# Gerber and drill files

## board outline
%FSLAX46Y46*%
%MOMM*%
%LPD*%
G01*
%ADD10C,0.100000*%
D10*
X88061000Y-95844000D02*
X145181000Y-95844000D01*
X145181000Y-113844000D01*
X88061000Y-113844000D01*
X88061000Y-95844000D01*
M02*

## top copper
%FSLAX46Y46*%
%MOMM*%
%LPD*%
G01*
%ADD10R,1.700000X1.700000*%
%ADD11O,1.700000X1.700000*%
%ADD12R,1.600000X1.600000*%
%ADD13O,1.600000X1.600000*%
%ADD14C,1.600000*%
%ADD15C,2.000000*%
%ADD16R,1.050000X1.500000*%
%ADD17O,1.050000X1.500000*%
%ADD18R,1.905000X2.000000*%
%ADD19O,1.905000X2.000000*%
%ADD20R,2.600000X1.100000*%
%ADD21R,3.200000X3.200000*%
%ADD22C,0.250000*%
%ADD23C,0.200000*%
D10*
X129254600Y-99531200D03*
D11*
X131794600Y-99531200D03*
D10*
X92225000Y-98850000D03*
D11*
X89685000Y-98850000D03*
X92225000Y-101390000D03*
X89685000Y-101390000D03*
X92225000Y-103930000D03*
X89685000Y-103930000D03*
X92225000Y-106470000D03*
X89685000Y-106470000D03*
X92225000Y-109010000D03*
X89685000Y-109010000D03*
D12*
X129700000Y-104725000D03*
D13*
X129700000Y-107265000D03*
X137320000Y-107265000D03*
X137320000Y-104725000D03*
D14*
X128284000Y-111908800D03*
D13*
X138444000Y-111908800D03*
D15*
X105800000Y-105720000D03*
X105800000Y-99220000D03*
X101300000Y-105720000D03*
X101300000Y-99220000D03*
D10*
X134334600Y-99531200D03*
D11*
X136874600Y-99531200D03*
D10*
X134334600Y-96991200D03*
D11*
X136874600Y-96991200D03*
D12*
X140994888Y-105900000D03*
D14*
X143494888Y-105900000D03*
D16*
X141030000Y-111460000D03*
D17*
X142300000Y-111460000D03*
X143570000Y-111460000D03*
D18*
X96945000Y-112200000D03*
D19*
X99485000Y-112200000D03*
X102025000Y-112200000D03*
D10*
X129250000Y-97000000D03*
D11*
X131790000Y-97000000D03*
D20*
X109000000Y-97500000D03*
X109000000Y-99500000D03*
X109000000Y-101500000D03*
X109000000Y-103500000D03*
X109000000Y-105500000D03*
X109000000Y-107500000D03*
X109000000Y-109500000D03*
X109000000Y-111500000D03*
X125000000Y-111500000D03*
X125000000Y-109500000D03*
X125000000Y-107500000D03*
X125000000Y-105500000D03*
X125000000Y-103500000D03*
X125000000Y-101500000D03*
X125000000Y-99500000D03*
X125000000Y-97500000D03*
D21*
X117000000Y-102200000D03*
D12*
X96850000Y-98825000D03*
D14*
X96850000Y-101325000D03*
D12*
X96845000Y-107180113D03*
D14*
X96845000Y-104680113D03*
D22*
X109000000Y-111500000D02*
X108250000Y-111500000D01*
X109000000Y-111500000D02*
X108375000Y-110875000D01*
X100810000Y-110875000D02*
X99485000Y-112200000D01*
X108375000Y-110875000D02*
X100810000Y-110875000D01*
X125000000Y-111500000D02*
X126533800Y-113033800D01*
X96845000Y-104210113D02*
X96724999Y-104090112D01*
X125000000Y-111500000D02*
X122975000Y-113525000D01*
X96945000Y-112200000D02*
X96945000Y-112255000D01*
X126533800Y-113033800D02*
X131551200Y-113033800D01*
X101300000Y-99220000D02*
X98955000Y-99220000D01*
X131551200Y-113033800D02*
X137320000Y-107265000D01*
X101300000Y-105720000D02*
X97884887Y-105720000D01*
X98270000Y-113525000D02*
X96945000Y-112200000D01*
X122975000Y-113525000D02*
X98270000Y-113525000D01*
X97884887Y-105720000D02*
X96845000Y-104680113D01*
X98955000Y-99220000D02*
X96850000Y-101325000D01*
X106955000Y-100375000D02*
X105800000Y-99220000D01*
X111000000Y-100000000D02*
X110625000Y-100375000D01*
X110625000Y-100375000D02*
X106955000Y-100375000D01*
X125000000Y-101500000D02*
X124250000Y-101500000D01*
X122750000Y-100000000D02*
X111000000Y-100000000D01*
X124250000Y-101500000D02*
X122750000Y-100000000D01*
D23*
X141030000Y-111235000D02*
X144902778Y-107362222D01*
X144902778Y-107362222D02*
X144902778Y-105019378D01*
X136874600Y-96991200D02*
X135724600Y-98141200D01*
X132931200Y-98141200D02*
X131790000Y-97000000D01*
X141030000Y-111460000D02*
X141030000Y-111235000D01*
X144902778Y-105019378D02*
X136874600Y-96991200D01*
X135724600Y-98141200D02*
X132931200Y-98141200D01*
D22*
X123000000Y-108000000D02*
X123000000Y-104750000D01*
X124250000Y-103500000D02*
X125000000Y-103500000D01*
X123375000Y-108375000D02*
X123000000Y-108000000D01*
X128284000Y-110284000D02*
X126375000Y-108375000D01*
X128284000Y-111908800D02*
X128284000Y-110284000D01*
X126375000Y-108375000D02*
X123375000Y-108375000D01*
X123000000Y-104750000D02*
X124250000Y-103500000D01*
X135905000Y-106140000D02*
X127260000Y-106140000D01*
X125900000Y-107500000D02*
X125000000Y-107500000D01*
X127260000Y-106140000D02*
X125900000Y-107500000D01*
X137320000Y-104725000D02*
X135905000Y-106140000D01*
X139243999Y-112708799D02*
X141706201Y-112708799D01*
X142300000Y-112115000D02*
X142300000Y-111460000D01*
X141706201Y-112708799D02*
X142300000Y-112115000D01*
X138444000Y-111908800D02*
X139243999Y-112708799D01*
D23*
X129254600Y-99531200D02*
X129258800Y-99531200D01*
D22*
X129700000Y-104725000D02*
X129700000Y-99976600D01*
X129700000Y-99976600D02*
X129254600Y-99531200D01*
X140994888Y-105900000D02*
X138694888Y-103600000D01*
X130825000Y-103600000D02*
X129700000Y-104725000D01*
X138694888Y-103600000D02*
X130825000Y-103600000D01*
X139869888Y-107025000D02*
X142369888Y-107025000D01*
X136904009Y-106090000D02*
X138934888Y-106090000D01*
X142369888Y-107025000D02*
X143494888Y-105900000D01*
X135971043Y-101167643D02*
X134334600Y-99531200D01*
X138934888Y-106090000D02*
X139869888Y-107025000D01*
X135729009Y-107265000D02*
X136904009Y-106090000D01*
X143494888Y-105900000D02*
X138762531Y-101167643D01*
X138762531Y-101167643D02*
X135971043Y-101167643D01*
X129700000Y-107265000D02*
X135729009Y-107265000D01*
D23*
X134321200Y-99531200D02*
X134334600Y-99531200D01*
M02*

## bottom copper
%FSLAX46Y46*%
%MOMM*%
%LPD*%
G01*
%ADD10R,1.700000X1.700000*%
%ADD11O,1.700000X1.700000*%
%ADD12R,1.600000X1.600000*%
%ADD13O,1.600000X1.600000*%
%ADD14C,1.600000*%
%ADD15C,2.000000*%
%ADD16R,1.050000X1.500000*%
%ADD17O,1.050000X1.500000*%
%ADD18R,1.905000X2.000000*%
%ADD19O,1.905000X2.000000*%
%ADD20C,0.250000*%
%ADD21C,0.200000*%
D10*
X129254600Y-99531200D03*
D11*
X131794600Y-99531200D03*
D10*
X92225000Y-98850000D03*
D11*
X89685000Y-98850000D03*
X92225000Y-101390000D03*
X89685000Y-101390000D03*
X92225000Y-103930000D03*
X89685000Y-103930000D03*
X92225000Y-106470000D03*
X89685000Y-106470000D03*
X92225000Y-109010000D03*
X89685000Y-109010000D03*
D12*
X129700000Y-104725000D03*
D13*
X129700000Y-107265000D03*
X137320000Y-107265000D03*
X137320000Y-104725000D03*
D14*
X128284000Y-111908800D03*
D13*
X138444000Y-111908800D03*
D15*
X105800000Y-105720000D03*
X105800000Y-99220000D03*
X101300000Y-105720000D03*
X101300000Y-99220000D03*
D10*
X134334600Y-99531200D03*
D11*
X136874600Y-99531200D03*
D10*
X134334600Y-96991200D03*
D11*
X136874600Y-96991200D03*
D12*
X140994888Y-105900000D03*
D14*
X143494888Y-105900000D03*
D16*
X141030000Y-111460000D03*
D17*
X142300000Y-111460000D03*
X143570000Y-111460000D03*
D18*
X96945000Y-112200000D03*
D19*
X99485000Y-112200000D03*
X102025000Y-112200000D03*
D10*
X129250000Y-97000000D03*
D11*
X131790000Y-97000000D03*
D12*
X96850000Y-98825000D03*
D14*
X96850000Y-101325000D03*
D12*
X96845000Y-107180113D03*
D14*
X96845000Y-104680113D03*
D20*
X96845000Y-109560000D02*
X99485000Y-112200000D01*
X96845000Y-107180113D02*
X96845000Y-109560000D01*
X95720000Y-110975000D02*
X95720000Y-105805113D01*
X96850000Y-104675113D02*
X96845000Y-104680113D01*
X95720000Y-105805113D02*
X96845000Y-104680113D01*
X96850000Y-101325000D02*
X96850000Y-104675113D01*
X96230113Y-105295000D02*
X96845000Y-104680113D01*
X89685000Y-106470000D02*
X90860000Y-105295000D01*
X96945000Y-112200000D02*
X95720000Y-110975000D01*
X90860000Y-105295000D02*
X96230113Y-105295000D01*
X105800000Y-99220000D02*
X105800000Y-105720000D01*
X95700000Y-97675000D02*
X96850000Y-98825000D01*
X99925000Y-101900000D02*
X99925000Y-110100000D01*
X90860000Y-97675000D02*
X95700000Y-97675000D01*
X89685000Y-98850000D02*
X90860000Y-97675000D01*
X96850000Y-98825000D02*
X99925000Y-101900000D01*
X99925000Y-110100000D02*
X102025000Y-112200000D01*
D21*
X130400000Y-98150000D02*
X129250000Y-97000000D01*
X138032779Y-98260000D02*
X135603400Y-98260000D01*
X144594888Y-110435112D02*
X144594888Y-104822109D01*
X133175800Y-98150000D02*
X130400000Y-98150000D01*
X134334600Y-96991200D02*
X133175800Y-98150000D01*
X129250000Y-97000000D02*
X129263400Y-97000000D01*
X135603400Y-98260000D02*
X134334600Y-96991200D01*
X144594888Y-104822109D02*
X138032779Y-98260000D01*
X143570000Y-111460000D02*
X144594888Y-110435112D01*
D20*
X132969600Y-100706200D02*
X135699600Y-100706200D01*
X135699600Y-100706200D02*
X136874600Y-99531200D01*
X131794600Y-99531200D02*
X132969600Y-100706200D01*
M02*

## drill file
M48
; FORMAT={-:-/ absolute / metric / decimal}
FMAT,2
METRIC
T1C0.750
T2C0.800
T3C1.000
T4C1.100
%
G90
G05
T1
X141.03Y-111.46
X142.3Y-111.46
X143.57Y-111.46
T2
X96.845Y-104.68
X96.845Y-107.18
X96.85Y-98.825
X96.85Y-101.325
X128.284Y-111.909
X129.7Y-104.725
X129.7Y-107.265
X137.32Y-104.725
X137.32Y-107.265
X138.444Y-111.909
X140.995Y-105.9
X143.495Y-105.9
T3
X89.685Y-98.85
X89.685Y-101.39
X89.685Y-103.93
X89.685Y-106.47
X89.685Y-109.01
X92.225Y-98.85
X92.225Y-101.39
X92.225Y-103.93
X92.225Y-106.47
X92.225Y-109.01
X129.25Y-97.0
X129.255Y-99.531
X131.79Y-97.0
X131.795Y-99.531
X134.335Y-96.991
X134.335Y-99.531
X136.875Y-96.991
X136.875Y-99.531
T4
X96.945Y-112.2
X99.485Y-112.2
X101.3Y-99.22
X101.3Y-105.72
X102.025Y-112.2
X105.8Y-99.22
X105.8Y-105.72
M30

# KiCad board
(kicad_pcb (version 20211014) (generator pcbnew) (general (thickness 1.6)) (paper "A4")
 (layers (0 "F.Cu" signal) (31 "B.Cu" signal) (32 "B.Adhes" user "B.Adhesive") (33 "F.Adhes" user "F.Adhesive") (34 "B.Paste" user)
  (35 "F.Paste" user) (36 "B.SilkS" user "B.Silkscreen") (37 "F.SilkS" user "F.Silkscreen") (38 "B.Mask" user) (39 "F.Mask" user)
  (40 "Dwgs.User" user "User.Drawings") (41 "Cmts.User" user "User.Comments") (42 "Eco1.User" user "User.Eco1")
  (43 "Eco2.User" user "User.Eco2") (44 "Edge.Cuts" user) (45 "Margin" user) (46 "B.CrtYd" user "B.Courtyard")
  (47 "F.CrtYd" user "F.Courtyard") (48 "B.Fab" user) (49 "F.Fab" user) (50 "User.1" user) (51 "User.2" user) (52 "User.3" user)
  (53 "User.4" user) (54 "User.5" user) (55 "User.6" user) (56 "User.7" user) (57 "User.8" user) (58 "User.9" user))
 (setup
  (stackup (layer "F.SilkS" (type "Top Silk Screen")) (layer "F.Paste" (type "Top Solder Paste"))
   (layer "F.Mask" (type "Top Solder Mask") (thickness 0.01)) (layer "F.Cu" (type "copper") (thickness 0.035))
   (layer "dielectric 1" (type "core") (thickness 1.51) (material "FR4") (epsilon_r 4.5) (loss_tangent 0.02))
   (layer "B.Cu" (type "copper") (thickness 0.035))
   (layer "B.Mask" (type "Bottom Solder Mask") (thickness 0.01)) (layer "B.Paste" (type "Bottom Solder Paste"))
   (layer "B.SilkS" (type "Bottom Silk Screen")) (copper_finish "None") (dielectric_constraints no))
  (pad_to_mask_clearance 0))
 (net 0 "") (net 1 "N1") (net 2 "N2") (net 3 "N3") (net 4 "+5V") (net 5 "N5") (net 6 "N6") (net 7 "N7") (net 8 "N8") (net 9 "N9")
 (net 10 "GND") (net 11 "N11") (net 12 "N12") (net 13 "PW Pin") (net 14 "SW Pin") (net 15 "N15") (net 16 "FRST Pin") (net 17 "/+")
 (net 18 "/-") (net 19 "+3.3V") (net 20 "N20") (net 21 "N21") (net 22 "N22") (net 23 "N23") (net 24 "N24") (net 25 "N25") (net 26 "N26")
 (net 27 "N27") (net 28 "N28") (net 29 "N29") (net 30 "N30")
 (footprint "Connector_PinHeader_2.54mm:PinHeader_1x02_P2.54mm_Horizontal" (layer "F.Cu") (at 129.2546 99.5312 90)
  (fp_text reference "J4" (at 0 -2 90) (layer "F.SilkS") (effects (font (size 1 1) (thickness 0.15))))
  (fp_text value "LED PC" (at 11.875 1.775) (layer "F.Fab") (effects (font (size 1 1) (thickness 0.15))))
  (pad "1" thru_hole rect (at 0 0 90) (size 1.7 1.7) (drill 1) (layers *.Cu *.Mask) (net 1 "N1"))
  (pad "2" thru_hole oval (at 0 2.54 90) (size 1.7 1.7) (drill 1) (layers *.Cu *.Mask) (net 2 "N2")))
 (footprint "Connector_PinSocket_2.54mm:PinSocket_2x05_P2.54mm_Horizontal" (layer "F.Cu") (at 92.225 98.85)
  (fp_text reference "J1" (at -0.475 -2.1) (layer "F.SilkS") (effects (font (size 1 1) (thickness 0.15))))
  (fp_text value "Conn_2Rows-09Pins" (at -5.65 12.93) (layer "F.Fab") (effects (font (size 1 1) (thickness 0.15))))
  (pad "1" thru_hole rect (at 0 0) (size 1.7 1.7) (drill 1) (layers *.Cu *.Mask) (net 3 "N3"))
  (pad "2" thru_hole oval (at -2.54 0) (size 1.7 1.7) (drill 1) (layers *.Cu *.Mask) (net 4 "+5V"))
  (pad "3" thru_hole oval (at 0 2.54) (size 1.7 1.7) (drill 1) (layers *.Cu *.Mask) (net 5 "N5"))
  (pad "4" thru_hole oval (at -2.54 2.54) (size 1.7 1.7) (drill 1) (layers *.Cu *.Mask) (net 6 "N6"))
  (pad "5" thru_hole oval (at 0 5.08) (size 1.7 1.7) (drill 1) (layers *.Cu *.Mask) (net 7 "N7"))
  (pad "6" thru_hole oval (at -2.54 5.08) (size 1.7 1.7) (drill 1) (layers *.Cu *.Mask) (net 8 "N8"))
  (pad "7" thru_hole oval (at 0 7.62) (size 1.7 1.7) (drill 1) (layers *.Cu *.Mask) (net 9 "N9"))
  (pad "8" thru_hole oval (at -2.54 7.62) (size 1.7 1.7) (drill 1) (layers *.Cu *.Mask) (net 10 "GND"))
  (pad "9" thru_hole oval (at 0 10.16) (size 1.7 1.7) (drill 1) (layers *.Cu *.Mask) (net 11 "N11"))
  (pad "10" thru_hole oval (at -2.54 10.16) (size 1.7 1.7) (drill 1) (layers *.Cu *.Mask)))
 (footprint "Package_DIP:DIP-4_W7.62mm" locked (layer "F.Cu") (at 129.7 104.725)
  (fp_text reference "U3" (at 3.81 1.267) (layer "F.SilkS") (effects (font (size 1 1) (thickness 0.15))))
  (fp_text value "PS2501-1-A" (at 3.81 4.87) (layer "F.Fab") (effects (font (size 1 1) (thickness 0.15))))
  (pad "1" thru_hole rect locked (at 0 0) (size 1.6 1.6) (drill 0.8) (layers *.Cu *.Mask) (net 1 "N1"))
  (pad "2" thru_hole oval locked (at 0 2.54) (size 1.6 1.6) (drill 0.8) (layers *.Cu *.Mask) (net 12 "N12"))
  (pad "3" thru_hole oval locked (at 7.62 2.54) (size 1.6 1.6) (drill 0.8) (layers *.Cu *.Mask) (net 10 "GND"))
  (pad "4" thru_hole oval locked (at 7.62 0) (size 1.6 1.6) (drill 0.8) (layers *.Cu *.Mask) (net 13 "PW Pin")))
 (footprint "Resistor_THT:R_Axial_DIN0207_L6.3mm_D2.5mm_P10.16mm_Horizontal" (layer "F.Cu") (at 128.284 111.9088)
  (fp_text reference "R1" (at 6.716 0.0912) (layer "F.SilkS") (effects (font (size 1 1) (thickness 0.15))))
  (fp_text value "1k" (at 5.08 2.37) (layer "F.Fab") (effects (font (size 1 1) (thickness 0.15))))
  (pad "1" thru_hole circle (at 0 0) (size 1.6 1.6) (drill 0.8) (layers *.Cu *.Mask) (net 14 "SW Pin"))
  (pad "2" thru_hole oval (at 10.16 0) (size 1.6 1.6) (drill 0.8) (layers *.Cu *.Mask) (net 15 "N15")))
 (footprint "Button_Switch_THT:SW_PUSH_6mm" (layer "F.Cu") (at 105.8 99.22 -90)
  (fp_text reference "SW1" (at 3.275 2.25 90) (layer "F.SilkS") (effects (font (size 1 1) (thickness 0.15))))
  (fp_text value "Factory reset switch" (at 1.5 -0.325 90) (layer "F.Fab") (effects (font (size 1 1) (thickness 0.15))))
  (pad "1" thru_hole circle (at 6.5 0) (size 2 2) (drill 1.1) (layers *.Cu *.Mask) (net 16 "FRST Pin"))
  (pad "1" thru_hole circle (at 0 0) (size 2 2) (drill 1.1) (layers *.Cu *.Mask) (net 16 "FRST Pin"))
  (pad "2" thru_hole circle (at 6.5 4.5) (size 2 2) (drill 1.1) (layers *.Cu *.Mask) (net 10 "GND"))
  (pad "2" thru_hole circle (at 0 4.5) (size 2 2) (drill 1.1) (layers *.Cu *.Mask) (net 10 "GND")))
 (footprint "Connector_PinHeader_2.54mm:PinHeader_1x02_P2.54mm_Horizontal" (layer "F.Cu") (at 134.3346 99.5312 90)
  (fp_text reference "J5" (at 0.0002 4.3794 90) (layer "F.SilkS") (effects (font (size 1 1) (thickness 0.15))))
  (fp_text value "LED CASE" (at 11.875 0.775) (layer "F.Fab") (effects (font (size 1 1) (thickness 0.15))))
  (pad "1" thru_hole rect (at 0 0 90) (size 1.7 1.7) (drill 1) (layers *.Cu *.Mask) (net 12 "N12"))
  (pad "2" thru_hole oval (at 0 2.54 90) (size 1.7 1.7) (drill 1) (layers *.Cu *.Mask) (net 2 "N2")))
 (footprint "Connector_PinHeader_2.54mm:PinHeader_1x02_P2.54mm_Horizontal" (layer "F.Cu") (at 134.3346 96.9912 90)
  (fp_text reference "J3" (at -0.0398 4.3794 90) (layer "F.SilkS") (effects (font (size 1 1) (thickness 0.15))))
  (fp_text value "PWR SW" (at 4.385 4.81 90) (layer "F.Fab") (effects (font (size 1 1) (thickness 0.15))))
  (pad "1" thru_hole rect (at 0 0 90) (size 1.7 1.7) (drill 1) (layers *.Cu *.Mask) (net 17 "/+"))
  (pad "2" thru_hole oval (at 0 2.54 90) (size 1.7 1.7) (drill 1) (layers *.Cu *.Mask) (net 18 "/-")))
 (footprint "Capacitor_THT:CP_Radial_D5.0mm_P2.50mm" (layer "F.Cu") (at 140.994888 105.9)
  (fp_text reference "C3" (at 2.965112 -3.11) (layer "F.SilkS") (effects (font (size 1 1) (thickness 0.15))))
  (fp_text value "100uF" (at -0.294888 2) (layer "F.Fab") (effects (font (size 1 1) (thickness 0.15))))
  (pad "1" thru_hole rect (at 0 0) (size 1.6 1.6) (drill 0.8) (layers *.Cu *.Mask) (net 1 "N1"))
  (pad "2" thru_hole circle (at 2.5 0) (size 1.6 1.6) (drill 0.8) (layers *.Cu *.Mask) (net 12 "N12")))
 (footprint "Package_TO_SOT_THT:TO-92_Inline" (layer "F.Cu") (at 141.03 111.46)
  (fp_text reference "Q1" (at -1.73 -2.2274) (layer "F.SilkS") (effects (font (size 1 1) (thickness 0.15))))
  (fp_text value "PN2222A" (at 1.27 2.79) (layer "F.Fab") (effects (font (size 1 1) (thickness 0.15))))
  (pad "1" thru_hole rect (at 0 0) (size 1.05 1.5) (drill 0.75) (layers *.Cu *.Mask) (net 18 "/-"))
  (pad "2" thru_hole oval (at 1.27 0) (size 1.05 1.5) (drill 0.75) (layers *.Cu *.Mask) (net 15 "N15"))
  (pad "3" thru_hole oval (at 2.54 0) (size 1.05 1.5) (drill 0.75) (layers *.Cu *.Mask) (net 17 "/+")))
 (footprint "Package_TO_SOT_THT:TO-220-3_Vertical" (layer "F.Cu") (at 96.945 112.2)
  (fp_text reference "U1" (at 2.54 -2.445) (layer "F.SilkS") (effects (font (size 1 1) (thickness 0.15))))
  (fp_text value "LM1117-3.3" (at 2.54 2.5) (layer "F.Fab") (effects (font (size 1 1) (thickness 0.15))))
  (pad "1" thru_hole rect (at 0 0) (size 1.905 2) (drill 1.1) (layers *.Cu *.Mask) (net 10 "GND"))
  (pad "2" thru_hole oval (at 2.54 0) (size 1.905 2) (drill 1.1) (layers *.Cu *.Mask) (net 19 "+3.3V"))
  (pad "3" thru_hole oval (at 5.08 0) (size 1.905 2) (drill 1.1) (layers *.Cu *.Mask) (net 4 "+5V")))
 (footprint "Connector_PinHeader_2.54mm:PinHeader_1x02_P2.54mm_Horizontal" (layer "F.Cu") (at 129.25 97 90)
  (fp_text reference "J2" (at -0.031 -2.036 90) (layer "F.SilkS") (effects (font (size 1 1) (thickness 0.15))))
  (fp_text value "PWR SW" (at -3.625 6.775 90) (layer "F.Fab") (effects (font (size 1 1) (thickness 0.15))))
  (pad "1" thru_hole rect (at 0 0 90) (size 1.7 1.7) (drill 1) (layers *.Cu *.Mask) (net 17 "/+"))
  (pad "2" thru_hole oval (at 0 2.54 90) (size 1.7 1.7) (drill 1) (layers *.Cu *.Mask) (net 18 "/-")))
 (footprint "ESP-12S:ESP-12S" (layer "F.Cu") (at 117 101)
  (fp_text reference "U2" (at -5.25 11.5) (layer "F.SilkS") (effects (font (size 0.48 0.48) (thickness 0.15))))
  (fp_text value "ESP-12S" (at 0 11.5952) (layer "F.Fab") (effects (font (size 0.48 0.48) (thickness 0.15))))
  (pad "1" smd rect locked (at -8 -3.5) (size 2.6 1.1) (layers "F.Cu" "F.Paste" "F.Mask") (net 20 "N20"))
  (pad "2" smd rect locked (at -8 -1.5) (size 2.6 1.1) (layers "F.Cu" "F.Paste" "F.Mask") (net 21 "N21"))
  (pad "3" smd rect locked (at -8 0.5) (size 2.6 1.1) (layers "F.Cu" "F.Paste" "F.Mask") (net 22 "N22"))
  (pad "4" smd rect locked (at -8 2.5) (size 2.6 1.1) (layers "F.Cu" "F.Paste" "F.Mask") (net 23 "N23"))
  (pad "5" smd rect locked (at -8 4.5) (size 2.6 1.1) (layers "F.Cu" "F.Paste" "F.Mask") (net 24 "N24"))
  (pad "6" smd rect locked (at -8 6.5) (size 2.6 1.1) (layers "F.Cu" "F.Paste" "F.Mask") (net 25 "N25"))
  (pad "7" smd rect locked (at -8 8.5) (size 2.6 1.1) (layers "F.Cu" "F.Paste" "F.Mask") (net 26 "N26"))
  (pad "8" smd rect locked (at -8 10.5) (size 2.6 1.1) (layers "F.Cu" "F.Paste" "F.Mask") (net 19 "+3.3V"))
  (pad "9" smd rect locked (at 8 10.5 180) (size 2.6 1.1) (layers "F.Cu" "F.Paste" "F.Mask") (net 10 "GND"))
  (pad "10" smd rect locked (at 8 8.5 180) (size 2.6 1.1) (layers "F.Cu" "F.Paste" "F.Mask") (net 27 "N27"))
  (pad "11" smd rect locked (at 8 6.5 180) (size 2.6 1.1) (layers "F.Cu" "F.Paste" "F.Mask") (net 13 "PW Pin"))
  (pad "12" smd rect locked (at 8 4.5 180) (size 2.6 1.1) (layers "F.Cu" "F.Paste" "F.Mask") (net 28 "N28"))
  (pad "13" smd rect locked (at 8 2.5 180) (size 2.6 1.1) (layers "F.Cu" "F.Paste" "F.Mask") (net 14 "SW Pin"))
  (pad "14" smd rect locked (at 8 0.5 180) (size 2.6 1.1) (layers "F.Cu" "F.Paste" "F.Mask") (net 16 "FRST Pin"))
  (pad "15" smd rect locked (at 8 -1.5 180) (size 2.6 1.1) (layers "F.Cu" "F.Paste" "F.Mask") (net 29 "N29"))
  (pad "16" smd rect locked (at 8 -3.5 180) (size 2.6 1.1) (layers "F.Cu" "F.Paste" "F.Mask") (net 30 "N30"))
  (pad "P$1" smd rect locked (at 0 1.2) (size 3.2 3.2) (layers "F.Cu"))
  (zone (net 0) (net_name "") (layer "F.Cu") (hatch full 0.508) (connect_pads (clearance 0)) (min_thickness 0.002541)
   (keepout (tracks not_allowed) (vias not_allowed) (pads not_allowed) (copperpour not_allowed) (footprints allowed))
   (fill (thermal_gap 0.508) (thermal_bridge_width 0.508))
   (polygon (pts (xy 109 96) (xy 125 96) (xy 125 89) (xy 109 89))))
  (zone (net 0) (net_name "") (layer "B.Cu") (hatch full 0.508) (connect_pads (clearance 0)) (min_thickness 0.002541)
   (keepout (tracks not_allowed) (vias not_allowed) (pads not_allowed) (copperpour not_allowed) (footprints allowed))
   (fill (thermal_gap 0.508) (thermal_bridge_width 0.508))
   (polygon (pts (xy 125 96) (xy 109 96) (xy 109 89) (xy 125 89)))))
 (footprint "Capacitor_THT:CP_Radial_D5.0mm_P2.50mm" (layer "F.Cu") (at 96.85 98.825 -90)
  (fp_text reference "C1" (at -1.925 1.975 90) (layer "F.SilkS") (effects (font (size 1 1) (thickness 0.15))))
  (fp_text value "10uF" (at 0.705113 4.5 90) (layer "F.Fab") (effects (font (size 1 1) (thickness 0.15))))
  (pad "1" thru_hole rect (at 0 0 270) (size 1.6 1.6) (drill 0.8) (layers *.Cu *.Mask) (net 4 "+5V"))
  (pad "2" thru_hole circle (at 2.5 0 270) (size 1.6 1.6) (drill 0.8) (layers *.Cu *.Mask) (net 10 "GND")))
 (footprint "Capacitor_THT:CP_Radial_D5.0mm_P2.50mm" (layer "F.Cu") (at 96.845 107.180113 90)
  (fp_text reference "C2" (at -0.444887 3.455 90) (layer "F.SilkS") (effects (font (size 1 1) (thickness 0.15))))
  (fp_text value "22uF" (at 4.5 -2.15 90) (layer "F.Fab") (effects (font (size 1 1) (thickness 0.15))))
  (pad "1" thru_hole rect (at 0 0 90) (size 1.6 1.6) (drill 0.8) (layers *.Cu *.Mask) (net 19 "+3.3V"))
  (pad "2" thru_hole circle (at 2.5 0 90) (size 1.6 1.6) (drill 0.8) (layers *.Cu *.Mask) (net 10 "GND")))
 (gr_rect (start 145.181 113.844) (end 88.061 95.844) (layer "Edge.Cuts") (width 0.1) (fill none))
 (segment (start 109 111.5) (end 108.25 111.5) (width 0.25) (layer "F.Cu") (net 19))
 (segment (start 109 111.5) (end 108.375 110.875) (width 0.25) (layer "F.Cu") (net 19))
 (segment (start 100.81 110.875) (end 99.485 112.2) (width 0.25) (layer "F.Cu") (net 19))
 (segment (start 108.375 110.875) (end 100.81 110.875) (width 0.25) (layer "F.Cu") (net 19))
 (segment (start 96.845 109.56) (end 99.485 112.2) (width 0.25) (layer "B.Cu") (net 19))
 (segment (start 96.845 107.180113) (end 96.845 109.56) (width 0.25) (layer "B.Cu") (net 19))
 (segment (start 125 111.5) (end 126.5338 113.0338) (width 0.25) (layer "F.Cu") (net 10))
 (segment (start 96.845 104.210113) (end 96.724999 104.090112) (width 0.25) (layer "F.Cu") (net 10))
 (segment (start 125 111.5) (end 122.975 113.525) (width 0.25) (layer "F.Cu") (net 10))
 (segment (start 96.945 112.2) (end 96.945 112.255) (width 0.25) (layer "F.Cu") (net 10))
 (segment (start 126.5338 113.0338) (end 131.5512 113.0338) (width 0.25) (layer "F.Cu") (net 10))
 (segment (start 101.3 99.22) (end 98.955 99.22) (width 0.25) (layer "F.Cu") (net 10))
 (segment (start 131.5512 113.0338) (end 137.32 107.265) (width 0.25) (layer "F.Cu") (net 10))
 (segment (start 101.3 105.72) (end 97.884887 105.72) (width 0.25) (layer "F.Cu") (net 10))
 (segment (start 98.27 113.525) (end 96.945 112.2) (width 0.25) (layer "F.Cu") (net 10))
 (segment (start 122.975 113.525) (end 98.27 113.525) (width 0.25) (layer "F.Cu") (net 10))
 (segment (start 97.884887 105.72) (end 96.845 104.680113) (width 0.25) (layer "F.Cu") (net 10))
 (segment (start 98.955 99.22) (end 96.85 101.325) (width 0.25) (layer "F.Cu") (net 10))
 (segment (start 95.72 110.975) (end 95.72 105.805113) (width 0.25) (layer "B.Cu") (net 10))
 (segment (start 96.85 104.675113) (end 96.845 104.680113) (width 0.25) (layer "B.Cu") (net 10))
 (segment (start 95.72 105.805113) (end 96.845 104.680113) (width 0.25) (layer "B.Cu") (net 10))
 (segment (start 96.85 101.325) (end 96.85 104.675113) (width 0.25) (layer "B.Cu") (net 10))
 (segment (start 96.230113 105.295) (end 96.845 104.680113) (width 0.25) (layer "B.Cu") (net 10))
 (segment (start 89.685 106.47) (end 90.86 105.295) (width 0.25) (layer "B.Cu") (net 10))
 (segment (start 96.945 112.2) (end 95.72 110.975) (width 0.25) (layer "B.Cu") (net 10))
 (segment (start 90.86 105.295) (end 96.230113 105.295) (width 0.25) (layer "B.Cu") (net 10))
 (segment (start 106.955 100.375) (end 105.8 99.22) (width 0.25) (layer "F.Cu") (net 16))
 (segment (start 111 100) (end 110.625 100.375) (width 0.25) (layer "F.Cu") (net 16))
 (segment (start 110.625 100.375) (end 106.955 100.375) (width 0.25) (layer "F.Cu") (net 16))
 (segment (start 125 101.5) (end 124.25 101.5) (width 0.25) (layer "F.Cu") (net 16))
 (segment (start 122.75 100) (end 111 100) (width 0.25) (layer "F.Cu") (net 16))
 (segment (start 124.25 101.5) (end 122.75 100) (width 0.25) (layer "F.Cu") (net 16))
 (segment (start 105.8 99.22) (end 105.8 105.72) (width 0.25) (layer "B.Cu") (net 16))
 (segment (start 95.7 97.675) (end 96.85 98.825) (width 0.25) (layer "B.Cu") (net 4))
 (segment (start 99.925 101.9) (end 99.925 110.1) (width 0.25) (layer "B.Cu") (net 4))
 (segment (start 90.86 97.675) (end 95.7 97.675) (width 0.25) (layer "B.Cu") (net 4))
 (segment (start 89.685 98.85) (end 90.86 97.675) (width 0.25) (layer "B.Cu") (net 4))
 (segment (start 96.85 98.825) (end 99.925 101.9) (width 0.25) (layer "B.Cu") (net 4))
 (segment (start 99.925 110.1) (end 102.025 112.2) (width 0.25) (layer "B.Cu") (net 4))
 (segment (start 130.4 98.15) (end 129.25 97) (width 0.2) (layer "B.Cu") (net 17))
 (segment (start 138.032779 98.26) (end 135.6034 98.26) (width 0.2) (layer "B.Cu") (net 17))
 (segment (start 144.594888 110.435112) (end 144.594888 104.822109) (width 0.2) (layer "B.Cu") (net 17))
 (segment (start 133.1758 98.15) (end 130.4 98.15) (width 0.2) (layer "B.Cu") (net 17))
 (segment (start 134.3346 96.9912) (end 133.1758 98.15) (width 0.2) (layer "B.Cu") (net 17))
 (segment (start 129.25 97) (end 129.2634 97) (width 0.2) (layer "B.Cu") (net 17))
 (segment (start 135.6034 98.26) (end 134.3346 96.9912) (width 0.2) (layer "B.Cu") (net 17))
 (segment (start 144.594888 104.822109) (end 138.032779 98.26) (width 0.2) (layer "B.Cu") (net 17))
 (segment (start 143.57 111.46) (end 144.594888 110.435112) (width 0.2) (layer "B.Cu") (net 17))
 (segment (start 141.03 111.235) (end 144.902778 107.362222) (width 0.2) (layer "F.Cu") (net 18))
 (segment (start 144.902778 107.362222) (end 144.902778 105.019378) (width 0.2) (layer "F.Cu") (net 18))
 (segment (start 136.8746 96.9912) (end 135.7246 98.1412) (width 0.2) (layer "F.Cu") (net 18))
 (segment (start 132.9312 98.1412) (end 131.79 97) (width 0.2) (layer "F.Cu") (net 18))
 (segment (start 141.03 111.46) (end 141.03 111.235) (width 0.2) (layer "F.Cu") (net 18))
 (segment (start 144.902778 105.019378) (end 136.8746 96.9912) (width 0.2) (layer "F.Cu") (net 18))
 (segment (start 135.7246 98.1412) (end 132.9312 98.1412) (width 0.2) (layer "F.Cu") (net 18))
 (segment (start 123 108) (end 123 104.75) (width 0.25) (layer "F.Cu") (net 14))
 (segment (start 124.25 103.5) (end 125 103.5) (width 0.25) (layer "F.Cu") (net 14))
 (segment (start 123.375 108.375) (end 123 108) (width 0.25) (layer "F.Cu") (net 14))
 (segment (start 128.284 110.284) (end 126.375 108.375) (width 0.25) (layer "F.Cu") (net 14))
 (segment (start 128.284 111.9088) (end 128.284 110.284) (width 0.25) (layer "F.Cu") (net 14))
 (segment (start 126.375 108.375) (end 123.375 108.375) (width 0.25) (layer "F.Cu") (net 14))
 (segment (start 123 104.75) (end 124.25 103.5) (width 0.25) (layer "F.Cu") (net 14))
 (segment (start 135.905 106.14) (end 127.26 106.14) (width 0.25) (layer "F.Cu") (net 13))
 (segment (start 125.9 107.5) (end 125 107.5) (width 0.25) (layer "F.Cu") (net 13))
 (segment (start 127.26 106.14) (end 125.9 107.5) (width 0.25) (layer "F.Cu") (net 13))
 (segment (start 137.32 104.725) (end 135.905 106.14) (width 0.25) (layer "F.Cu") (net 13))
 (segment (start 139.243999 112.708799) (end 141.706201 112.708799) (width 0.25) (layer "F.Cu") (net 15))
 (segment (start 142.3 112.115) (end 142.3 111.46) (width 0.25) (layer "F.Cu") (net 15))
 (segment (start 141.706201 112.708799) (end 142.3 112.115) (width 0.25) (layer "F.Cu") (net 15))
 (segment (start 138.444 111.9088) (end 139.243999 112.708799) (width 0.25) (layer "F.Cu") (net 15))
 (segment (start 129.2546 99.5312) (end 129.2588 99.5312) (width 0.2) (layer "F.Cu") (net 1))
 (segment (start 129.7 104.725) (end 129.7 99.9766) (width 0.25) (layer "F.Cu") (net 1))
 (segment (start 129.7 99.9766) (end 129.2546 99.5312) (width 0.25) (layer "F.Cu") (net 1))
 (segment (start 140.994888 105.9) (end 138.694888 103.6) (width 0.25) (layer "F.Cu") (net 1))
 (segment (start 130.825 103.6) (end 129.7 104.725) (width 0.25) (layer "F.Cu") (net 1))
 (segment (start 138.694888 103.6) (end 130.825 103.6) (width 0.25) (layer "F.Cu") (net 1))
 (segment (start 139.869888 107.025) (end 142.369888 107.025) (width 0.25) (layer "F.Cu") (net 12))
 (segment (start 136.904009 106.09) (end 138.934888 106.09) (width 0.25) (layer "F.Cu") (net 12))
 (segment (start 142.369888 107.025) (end 143.494888 105.9) (width 0.25) (layer "F.Cu") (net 12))
 (segment (start 135.971043 101.167643) (end 134.3346 99.5312) (width 0.25) (layer "F.Cu") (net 12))
 (segment (start 138.934888 106.09) (end 139.869888 107.025) (width 0.25) (layer "F.Cu") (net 12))
 (segment (start 135.729009 107.265) (end 136.904009 106.09) (width 0.25) (layer "F.Cu") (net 12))
 (segment (start 143.494888 105.9) (end 138.762531 101.167643) (width 0.25) (layer "F.Cu") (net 12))
 (segment (start 138.762531 101.167643) (end 135.971043 101.167643) (width 0.25) (layer "F.Cu") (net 12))
 (segment (start 129.7 107.265) (end 135.729009 107.265) (width 0.25) (layer "F.Cu") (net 12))
 (segment (start 134.3212 99.5312) (end 134.3346 99.5312) (width 0.2) (layer "F.Cu") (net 12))
 (segment (start 132.9696 100.7062) (end 135.6996 100.7062) (width 0.25) (layer "B.Cu") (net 2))
 (segment (start 135.6996 100.7062) (end 136.8746 99.5312) (width 0.25) (layer "B.Cu") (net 2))
 (segment (start 131.7946 99.5312) (end 132.9696 100.7062) (width 0.25) (layer "B.Cu") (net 2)))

